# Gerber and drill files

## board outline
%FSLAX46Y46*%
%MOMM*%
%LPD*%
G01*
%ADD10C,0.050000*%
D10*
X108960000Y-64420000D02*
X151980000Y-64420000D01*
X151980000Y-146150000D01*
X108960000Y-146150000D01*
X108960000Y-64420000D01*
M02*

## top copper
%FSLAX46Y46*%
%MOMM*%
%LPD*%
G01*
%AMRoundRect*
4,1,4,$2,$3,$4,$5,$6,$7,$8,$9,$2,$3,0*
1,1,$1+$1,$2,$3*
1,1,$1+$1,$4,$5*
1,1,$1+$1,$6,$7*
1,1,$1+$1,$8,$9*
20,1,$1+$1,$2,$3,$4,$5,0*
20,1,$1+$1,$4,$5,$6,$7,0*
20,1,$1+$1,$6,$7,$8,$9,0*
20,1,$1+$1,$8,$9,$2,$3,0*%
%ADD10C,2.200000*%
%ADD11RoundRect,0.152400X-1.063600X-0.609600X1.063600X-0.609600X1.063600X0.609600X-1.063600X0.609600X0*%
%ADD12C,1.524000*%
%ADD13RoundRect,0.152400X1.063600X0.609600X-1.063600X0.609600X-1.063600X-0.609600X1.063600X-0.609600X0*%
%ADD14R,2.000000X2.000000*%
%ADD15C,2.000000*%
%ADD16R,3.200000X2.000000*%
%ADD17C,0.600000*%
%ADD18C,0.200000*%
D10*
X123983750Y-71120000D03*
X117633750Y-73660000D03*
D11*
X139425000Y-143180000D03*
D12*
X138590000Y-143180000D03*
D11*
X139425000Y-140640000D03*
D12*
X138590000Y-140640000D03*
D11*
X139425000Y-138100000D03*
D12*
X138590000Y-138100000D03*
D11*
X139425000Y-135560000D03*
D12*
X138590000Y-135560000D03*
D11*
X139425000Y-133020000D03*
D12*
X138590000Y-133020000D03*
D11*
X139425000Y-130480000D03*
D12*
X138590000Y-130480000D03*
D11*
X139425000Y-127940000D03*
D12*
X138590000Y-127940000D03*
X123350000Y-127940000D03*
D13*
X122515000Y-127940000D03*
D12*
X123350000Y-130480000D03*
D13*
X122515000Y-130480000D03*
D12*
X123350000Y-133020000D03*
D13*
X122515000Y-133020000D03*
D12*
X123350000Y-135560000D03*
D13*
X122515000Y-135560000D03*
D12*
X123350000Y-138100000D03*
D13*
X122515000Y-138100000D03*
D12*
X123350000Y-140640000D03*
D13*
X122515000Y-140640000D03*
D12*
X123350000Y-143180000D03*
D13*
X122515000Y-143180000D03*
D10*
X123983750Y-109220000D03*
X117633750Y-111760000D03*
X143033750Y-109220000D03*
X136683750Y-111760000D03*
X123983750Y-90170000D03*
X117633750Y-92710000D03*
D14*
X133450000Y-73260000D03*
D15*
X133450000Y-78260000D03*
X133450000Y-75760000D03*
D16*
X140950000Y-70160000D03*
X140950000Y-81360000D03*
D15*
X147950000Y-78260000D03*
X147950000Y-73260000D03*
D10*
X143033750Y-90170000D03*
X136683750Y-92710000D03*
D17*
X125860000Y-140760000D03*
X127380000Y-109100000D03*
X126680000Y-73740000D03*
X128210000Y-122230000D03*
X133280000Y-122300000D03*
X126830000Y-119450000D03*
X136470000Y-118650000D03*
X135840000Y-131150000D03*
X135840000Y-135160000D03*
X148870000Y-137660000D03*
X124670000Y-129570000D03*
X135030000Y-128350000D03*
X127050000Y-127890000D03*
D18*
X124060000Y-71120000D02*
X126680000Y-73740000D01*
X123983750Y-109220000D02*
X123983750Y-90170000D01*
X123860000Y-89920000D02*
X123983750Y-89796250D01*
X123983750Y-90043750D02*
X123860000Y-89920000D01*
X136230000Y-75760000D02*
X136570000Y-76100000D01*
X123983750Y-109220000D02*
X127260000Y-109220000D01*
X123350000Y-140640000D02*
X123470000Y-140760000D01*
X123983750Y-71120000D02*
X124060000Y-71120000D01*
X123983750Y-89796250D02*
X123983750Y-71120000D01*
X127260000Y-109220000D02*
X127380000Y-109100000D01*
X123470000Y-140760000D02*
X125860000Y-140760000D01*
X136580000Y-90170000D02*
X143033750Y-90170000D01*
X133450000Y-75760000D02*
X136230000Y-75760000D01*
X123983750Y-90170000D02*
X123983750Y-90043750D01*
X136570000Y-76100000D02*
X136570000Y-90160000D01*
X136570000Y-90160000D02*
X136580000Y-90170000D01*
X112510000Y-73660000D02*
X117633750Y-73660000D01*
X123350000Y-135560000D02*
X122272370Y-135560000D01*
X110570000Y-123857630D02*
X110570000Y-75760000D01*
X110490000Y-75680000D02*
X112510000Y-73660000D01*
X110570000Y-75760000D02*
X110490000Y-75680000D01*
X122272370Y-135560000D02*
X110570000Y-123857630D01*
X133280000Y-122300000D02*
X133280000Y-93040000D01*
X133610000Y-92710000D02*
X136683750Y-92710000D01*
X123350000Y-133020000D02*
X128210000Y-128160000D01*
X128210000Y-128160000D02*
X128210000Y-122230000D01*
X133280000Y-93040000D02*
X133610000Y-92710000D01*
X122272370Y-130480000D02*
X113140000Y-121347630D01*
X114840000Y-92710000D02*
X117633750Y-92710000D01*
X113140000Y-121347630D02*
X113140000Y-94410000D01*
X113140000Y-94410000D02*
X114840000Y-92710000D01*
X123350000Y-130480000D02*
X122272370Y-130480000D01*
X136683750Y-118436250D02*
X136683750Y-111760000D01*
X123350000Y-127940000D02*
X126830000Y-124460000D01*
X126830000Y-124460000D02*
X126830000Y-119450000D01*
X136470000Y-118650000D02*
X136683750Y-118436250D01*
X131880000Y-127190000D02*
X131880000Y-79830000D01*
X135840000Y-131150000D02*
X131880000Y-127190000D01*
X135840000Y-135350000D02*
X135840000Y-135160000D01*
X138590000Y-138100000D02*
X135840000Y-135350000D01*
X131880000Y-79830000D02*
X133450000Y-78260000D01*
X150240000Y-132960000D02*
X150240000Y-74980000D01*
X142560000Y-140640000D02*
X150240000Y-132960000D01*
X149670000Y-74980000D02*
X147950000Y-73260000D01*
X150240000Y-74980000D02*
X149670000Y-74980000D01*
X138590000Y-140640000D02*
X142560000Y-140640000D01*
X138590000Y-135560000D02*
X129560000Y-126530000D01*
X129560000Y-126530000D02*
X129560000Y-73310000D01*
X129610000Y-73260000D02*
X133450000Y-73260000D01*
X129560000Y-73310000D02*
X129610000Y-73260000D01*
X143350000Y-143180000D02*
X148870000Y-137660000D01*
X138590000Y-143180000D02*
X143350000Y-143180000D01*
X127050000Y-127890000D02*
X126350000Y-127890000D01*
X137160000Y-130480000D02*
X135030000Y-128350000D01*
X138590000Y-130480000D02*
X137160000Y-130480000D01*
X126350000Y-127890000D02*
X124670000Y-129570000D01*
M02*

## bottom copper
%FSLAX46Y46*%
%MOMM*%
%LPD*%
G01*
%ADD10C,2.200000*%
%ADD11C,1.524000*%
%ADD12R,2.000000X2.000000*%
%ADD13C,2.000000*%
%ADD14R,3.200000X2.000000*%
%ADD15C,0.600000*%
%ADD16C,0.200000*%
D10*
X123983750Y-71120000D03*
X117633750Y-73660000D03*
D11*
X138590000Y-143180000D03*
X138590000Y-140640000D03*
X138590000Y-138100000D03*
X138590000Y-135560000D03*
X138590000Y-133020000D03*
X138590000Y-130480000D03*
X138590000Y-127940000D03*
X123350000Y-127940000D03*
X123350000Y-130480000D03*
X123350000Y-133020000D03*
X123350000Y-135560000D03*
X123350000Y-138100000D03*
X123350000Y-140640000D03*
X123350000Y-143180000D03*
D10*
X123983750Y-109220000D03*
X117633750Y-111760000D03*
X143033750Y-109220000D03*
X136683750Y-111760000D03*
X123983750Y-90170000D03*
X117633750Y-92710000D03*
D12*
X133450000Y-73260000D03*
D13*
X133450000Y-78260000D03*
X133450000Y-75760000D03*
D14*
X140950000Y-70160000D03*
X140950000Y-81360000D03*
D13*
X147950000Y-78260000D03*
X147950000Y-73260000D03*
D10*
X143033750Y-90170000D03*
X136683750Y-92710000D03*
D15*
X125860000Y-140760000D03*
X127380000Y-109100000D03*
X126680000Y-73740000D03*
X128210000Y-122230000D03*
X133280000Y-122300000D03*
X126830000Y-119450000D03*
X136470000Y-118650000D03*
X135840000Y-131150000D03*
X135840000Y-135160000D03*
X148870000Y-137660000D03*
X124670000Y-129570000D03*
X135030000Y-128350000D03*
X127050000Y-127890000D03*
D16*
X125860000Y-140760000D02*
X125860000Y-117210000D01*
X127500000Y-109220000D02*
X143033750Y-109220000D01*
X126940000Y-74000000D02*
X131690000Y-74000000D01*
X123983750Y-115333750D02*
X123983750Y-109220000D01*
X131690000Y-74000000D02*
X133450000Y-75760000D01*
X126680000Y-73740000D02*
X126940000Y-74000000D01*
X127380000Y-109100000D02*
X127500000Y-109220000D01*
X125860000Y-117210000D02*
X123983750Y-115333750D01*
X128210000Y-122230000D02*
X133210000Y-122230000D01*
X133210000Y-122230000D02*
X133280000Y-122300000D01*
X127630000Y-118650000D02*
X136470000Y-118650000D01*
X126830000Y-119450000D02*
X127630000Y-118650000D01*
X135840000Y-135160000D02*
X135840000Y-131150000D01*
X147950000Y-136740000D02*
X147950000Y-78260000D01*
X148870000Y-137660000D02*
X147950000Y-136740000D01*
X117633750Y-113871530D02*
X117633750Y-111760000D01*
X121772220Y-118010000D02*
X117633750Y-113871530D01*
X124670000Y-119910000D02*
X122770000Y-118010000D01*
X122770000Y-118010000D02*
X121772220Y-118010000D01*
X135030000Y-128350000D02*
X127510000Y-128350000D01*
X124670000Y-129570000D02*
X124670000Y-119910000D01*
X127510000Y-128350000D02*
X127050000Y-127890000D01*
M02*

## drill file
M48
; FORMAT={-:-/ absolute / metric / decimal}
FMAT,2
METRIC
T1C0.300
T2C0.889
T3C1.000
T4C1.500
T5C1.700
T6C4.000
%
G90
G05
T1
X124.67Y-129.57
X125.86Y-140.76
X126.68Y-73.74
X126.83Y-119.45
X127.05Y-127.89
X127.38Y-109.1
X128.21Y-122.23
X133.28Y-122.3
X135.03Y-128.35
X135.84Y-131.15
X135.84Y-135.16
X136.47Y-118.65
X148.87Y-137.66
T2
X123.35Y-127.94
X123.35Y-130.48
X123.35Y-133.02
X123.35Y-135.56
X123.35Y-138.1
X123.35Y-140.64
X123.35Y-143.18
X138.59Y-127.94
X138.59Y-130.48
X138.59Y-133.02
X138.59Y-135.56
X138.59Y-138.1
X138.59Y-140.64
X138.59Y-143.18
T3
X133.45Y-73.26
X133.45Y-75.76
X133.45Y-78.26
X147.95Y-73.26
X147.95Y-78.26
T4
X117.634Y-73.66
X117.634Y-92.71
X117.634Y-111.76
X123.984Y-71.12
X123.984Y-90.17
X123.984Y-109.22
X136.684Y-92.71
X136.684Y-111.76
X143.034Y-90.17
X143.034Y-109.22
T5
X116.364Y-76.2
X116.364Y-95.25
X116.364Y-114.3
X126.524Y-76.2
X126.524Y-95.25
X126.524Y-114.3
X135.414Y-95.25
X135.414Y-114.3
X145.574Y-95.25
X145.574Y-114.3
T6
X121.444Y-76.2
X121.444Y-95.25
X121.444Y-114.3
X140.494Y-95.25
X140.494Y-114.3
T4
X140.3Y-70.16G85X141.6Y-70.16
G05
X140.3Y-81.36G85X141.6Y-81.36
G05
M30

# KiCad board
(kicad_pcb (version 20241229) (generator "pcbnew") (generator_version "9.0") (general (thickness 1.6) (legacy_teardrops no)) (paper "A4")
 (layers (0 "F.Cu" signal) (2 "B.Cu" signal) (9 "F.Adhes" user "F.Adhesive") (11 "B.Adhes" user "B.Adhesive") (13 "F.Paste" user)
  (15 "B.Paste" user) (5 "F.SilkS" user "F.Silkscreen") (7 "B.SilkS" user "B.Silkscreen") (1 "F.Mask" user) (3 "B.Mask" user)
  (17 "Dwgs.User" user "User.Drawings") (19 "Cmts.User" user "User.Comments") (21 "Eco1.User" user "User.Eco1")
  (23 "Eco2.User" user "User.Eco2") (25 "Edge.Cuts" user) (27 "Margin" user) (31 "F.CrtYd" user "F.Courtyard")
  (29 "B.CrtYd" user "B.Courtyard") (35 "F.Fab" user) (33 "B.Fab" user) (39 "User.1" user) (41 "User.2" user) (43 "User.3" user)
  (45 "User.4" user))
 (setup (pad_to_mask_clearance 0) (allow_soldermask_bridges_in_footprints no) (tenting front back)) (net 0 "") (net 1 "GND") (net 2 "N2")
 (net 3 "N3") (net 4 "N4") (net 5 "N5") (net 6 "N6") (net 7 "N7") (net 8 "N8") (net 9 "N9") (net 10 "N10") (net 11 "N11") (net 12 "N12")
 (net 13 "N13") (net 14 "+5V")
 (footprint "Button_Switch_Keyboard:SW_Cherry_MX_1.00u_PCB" (layer "F.Cu") (at 123.98375 71.12)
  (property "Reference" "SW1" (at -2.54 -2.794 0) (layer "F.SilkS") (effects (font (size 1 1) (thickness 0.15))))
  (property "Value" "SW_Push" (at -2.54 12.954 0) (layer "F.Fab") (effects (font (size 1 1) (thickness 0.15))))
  (pad "" np_thru_hole circle (at -7.62 5.08) (size 1.7 1.7) (drill 1.7) (layers "*.Cu" "*.Mask"))
  (pad "" np_thru_hole circle (at -2.54 5.08) (size 4 4) (drill 4) (layers "*.Cu" "*.Mask"))
  (pad "" np_thru_hole circle (at 2.54 5.08) (size 1.7 1.7) (drill 1.7) (layers "*.Cu" "*.Mask"))
  (pad "1" thru_hole circle (at 0 0) (size 2.2 2.2) (drill 1.5) (layers "*.Cu" "*.Mask") (remove_unused_layers no) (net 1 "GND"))
  (pad "2" thru_hole circle (at -6.35 2.54) (size 2.2 2.2) (drill 1.5) (layers "*.Cu" "*.Mask") (remove_unused_layers no) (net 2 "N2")))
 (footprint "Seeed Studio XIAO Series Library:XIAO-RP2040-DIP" (layer "F.Cu") (at 130.97 135.56 180)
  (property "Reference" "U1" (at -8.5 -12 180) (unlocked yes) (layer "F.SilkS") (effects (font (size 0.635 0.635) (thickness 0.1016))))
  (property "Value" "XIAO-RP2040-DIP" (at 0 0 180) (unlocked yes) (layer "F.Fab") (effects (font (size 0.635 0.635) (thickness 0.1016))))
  (pad "1" smd roundrect (at -8.455 -7.62) (size 2.432 1.524) (layers "F.Cu" "F.Mask") (roundrect_rratio 0.1) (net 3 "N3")
   (thermal_bridge_angle 45))
  (pad "1" thru_hole circle (at -7.62 -7.62) (size 1.524 1.524) (drill 0.889) (layers "*.Cu" "*.Mask") (remove_unused_layers no)
   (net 3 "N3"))
  (pad "2" smd roundrect (at -8.455 -5.08) (size 2.432 1.524) (layers "F.Cu" "F.Mask") (roundrect_rratio 0.1) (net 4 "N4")
   (thermal_bridge_angle 45))
  (pad "2" thru_hole circle (at -7.62 -5.08) (size 1.524 1.524) (drill 0.889) (layers "*.Cu" "*.Mask") (remove_unused_layers no)
   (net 4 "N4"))
  (pad "3" smd roundrect (at -8.455 -2.54) (size 2.432 1.524) (layers "F.Cu" "F.Mask") (roundrect_rratio 0.1) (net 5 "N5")
   (thermal_bridge_angle 45))
  (pad "3" thru_hole circle (at -7.62 -2.54) (size 1.524 1.524) (drill 0.889) (layers "*.Cu" "*.Mask") (remove_unused_layers no)
   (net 5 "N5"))
  (pad "4" smd roundrect (at -8.455 0) (size 2.432 1.524) (layers "F.Cu" "F.Mask") (roundrect_rratio 0.1) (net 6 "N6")
   (thermal_bridge_angle 45))
  (pad "4" thru_hole circle (at -7.62 0) (size 1.524 1.524) (drill 0.889) (layers "*.Cu" "*.Mask") (remove_unused_layers no) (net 6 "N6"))
  (pad "5" smd roundrect (at -8.455 2.54) (size 2.432 1.524) (layers "F.Cu" "F.Mask") (roundrect_rratio 0.1) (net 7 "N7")
   (thermal_bridge_angle 45))
  (pad "5" thru_hole circle (at -7.62 2.54) (size 1.524 1.524) (drill 0.889) (layers "*.Cu" "*.Mask") (remove_unused_layers no) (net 7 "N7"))
  (pad "6" smd roundrect (at -8.455 5.08) (size 2.432 1.524) (layers "F.Cu" "F.Mask") (roundrect_rratio 0.1) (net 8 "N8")
   (thermal_bridge_angle 45))
  (pad "6" thru_hole circle (at -7.62 5.08) (size 1.524 1.524) (drill 0.889) (layers "*.Cu" "*.Mask") (remove_unused_layers no) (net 8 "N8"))
  (pad "7" smd roundrect (at -8.455 7.62) (size 2.432 1.524) (layers "F.Cu" "F.Mask") (roundrect_rratio 0.1) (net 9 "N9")
   (thermal_bridge_angle 45))
  (pad "7" thru_hole circle (at -7.62 7.62) (size 1.524 1.524) (drill 0.889) (layers "*.Cu" "*.Mask") (remove_unused_layers no) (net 9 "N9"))
  (pad "8" thru_hole circle (at 7.62 7.62 180) (size 1.524 1.524) (drill 0.889) (layers "*.Cu" "*.Mask") (remove_unused_layers no)
   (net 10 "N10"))
  (pad "8" smd roundrect (at 8.455 7.62 180) (size 2.432 1.524) (layers "F.Cu" "F.Mask") (roundrect_rratio 0.1) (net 10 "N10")
   (thermal_bridge_angle 45))
  (pad "9" thru_hole circle (at 7.62 5.08 180) (size 1.524 1.524) (drill 0.889) (layers "*.Cu" "*.Mask") (remove_unused_layers no)
   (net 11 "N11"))
  (pad "9" smd roundrect (at 8.455 5.08 180) (size 2.432 1.524) (layers "F.Cu" "F.Mask") (roundrect_rratio 0.1) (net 11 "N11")
   (thermal_bridge_angle 45))
  (pad "10" thru_hole circle (at 7.62 2.54 180) (size 1.524 1.524) (drill 0.889) (layers "*.Cu" "*.Mask") (remove_unused_layers no)
   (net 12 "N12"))
  (pad "10" smd roundrect (at 8.455 2.54 180) (size 2.432 1.524) (layers "F.Cu" "F.Mask") (roundrect_rratio 0.1) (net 12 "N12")
   (thermal_bridge_angle 45))
  (pad "11" thru_hole circle (at 7.62 0 180) (size 1.524 1.524) (drill 0.889) (layers "*.Cu" "*.Mask") (remove_unused_layers no)
   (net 2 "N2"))
  (pad "11" smd roundrect (at 8.455 0 180) (size 2.432 1.524) (layers "F.Cu" "F.Mask") (roundrect_rratio 0.1) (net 2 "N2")
   (thermal_bridge_angle 45))
  (pad "12" thru_hole circle (at 7.62 -2.54 180) (size 1.524 1.524) (drill 0.889) (layers "*.Cu" "*.Mask") (remove_unused_layers no)
   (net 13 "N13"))
  (pad "12" smd roundrect (at 8.455 -2.54 180) (size 2.432 1.524) (layers "F.Cu" "F.Mask") (roundrect_rratio 0.1) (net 13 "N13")
   (thermal_bridge_angle 45))
  (pad "13" thru_hole circle (at 7.62 -5.08 180) (size 1.524 1.524) (drill 0.889) (layers "*.Cu" "*.Mask") (remove_unused_layers no)
   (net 1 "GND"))
  (pad "13" smd roundrect (at 8.455 -5.08 180) (size 2.432 1.524) (layers "F.Cu" "F.Mask") (roundrect_rratio 0.1) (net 1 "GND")
   (thermal_bridge_angle 45))
  (pad "14" thru_hole circle (at 7.62 -7.62 180) (size 1.524 1.524) (drill 0.889) (layers "*.Cu" "*.Mask") (remove_unused_layers no)
   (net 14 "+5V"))
  (pad "14" smd roundrect (at 8.455 -7.62 180) (size 2.432 1.524) (layers "F.Cu" "F.Mask") (roundrect_rratio 0.1) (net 14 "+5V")
   (thermal_bridge_angle 45)))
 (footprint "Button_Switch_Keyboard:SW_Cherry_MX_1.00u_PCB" (layer "F.Cu") (at 123.98375 109.22)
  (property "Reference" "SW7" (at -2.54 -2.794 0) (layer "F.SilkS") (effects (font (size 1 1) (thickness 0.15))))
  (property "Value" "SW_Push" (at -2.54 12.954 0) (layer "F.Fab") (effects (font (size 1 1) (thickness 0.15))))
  (pad "" np_thru_hole circle (at -7.62 5.08) (size 1.7 1.7) (drill 1.7) (layers "*.Cu" "*.Mask"))
  (pad "" np_thru_hole circle (at -2.54 5.08) (size 4 4) (drill 4) (layers "*.Cu" "*.Mask"))
  (pad "" np_thru_hole circle (at 2.54 5.08) (size 1.7 1.7) (drill 1.7) (layers "*.Cu" "*.Mask"))
  (pad "1" thru_hole circle (at 0 0) (size 2.2 2.2) (drill 1.5) (layers "*.Cu" "*.Mask") (remove_unused_layers no) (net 1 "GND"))
  (pad "2" thru_hole circle (at -6.35 2.54) (size 2.2 2.2) (drill 1.5) (layers "*.Cu" "*.Mask") (remove_unused_layers no) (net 8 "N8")))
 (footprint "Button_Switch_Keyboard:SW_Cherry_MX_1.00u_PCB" (layer "F.Cu") (at 143.03375 109.22)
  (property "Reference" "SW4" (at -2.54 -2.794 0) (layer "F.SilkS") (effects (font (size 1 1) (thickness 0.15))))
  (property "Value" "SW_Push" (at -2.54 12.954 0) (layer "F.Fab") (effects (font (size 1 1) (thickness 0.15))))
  (pad "" np_thru_hole circle (at -7.62 5.08) (size 1.7 1.7) (drill 1.7) (layers "*.Cu" "*.Mask"))
  (pad "" np_thru_hole circle (at -2.54 5.08) (size 4 4) (drill 4) (layers "*.Cu" "*.Mask"))
  (pad "" np_thru_hole circle (at 2.54 5.08) (size 1.7 1.7) (drill 1.7) (layers "*.Cu" "*.Mask"))
  (pad "1" thru_hole circle (at 0 0) (size 2.2 2.2) (drill 1.5) (layers "*.Cu" "*.Mask") (remove_unused_layers no) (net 1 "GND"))
  (pad "2" thru_hole circle (at -6.35 2.54) (size 2.2 2.2) (drill 1.5) (layers "*.Cu" "*.Mask") (remove_unused_layers no) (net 10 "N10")))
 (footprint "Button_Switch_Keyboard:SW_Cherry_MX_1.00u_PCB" (layer "F.Cu") (at 123.98375 90.17)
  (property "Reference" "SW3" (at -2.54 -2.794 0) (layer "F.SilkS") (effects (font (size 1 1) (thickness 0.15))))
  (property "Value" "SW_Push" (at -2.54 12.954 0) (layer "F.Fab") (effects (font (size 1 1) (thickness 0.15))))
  (pad "" np_thru_hole circle (at -7.62 5.08) (size 1.7 1.7) (drill 1.7) (layers "*.Cu" "*.Mask"))
  (pad "" np_thru_hole circle (at -2.54 5.08) (size 4 4) (drill 4) (layers "*.Cu" "*.Mask"))
  (pad "" np_thru_hole circle (at 2.54 5.08) (size 1.7 1.7) (drill 1.7) (layers "*.Cu" "*.Mask"))
  (pad "1" thru_hole circle (at 0 0) (size 2.2 2.2) (drill 1.5) (layers "*.Cu" "*.Mask") (remove_unused_layers no) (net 1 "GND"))
  (pad "2" thru_hole circle (at -6.35 2.54) (size 2.2 2.2) (drill 1.5) (layers "*.Cu" "*.Mask") (remove_unused_layers no) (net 11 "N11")))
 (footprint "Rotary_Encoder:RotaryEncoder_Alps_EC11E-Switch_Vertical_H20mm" (layer "F.Cu") (at 133.45 73.26)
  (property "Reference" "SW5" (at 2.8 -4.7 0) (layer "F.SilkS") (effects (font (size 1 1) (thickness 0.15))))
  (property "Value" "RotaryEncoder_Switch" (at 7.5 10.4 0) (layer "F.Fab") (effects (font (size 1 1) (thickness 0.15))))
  (pad "A" thru_hole rect (at 0 0) (size 2 2) (drill 1) (layers "*.Cu" "*.Mask") (remove_unused_layers no) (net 6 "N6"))
  (pad "B" thru_hole circle (at 0 5) (size 2 2) (drill 1) (layers "*.Cu" "*.Mask") (remove_unused_layers no) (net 5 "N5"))
  (pad "C" thru_hole circle (at 0 2.5) (size 2 2) (drill 1) (layers "*.Cu" "*.Mask") (remove_unused_layers no) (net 1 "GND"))
  (pad "MP" thru_hole rect (at 7.5 -3.1) (size 3.2 2) (drill oval 2.8 1.5) (layers "*.Cu" "*.Mask") (remove_unused_layers no))
  (pad "MP" thru_hole rect (at 7.5 8.1) (size 3.2 2) (drill oval 2.8 1.5) (layers "*.Cu" "*.Mask") (remove_unused_layers no))
  (pad "S1" thru_hole circle (at 14.5 5) (size 2 2) (drill 1) (layers "*.Cu" "*.Mask") (remove_unused_layers no) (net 3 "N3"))
  (pad "S2" thru_hole circle (at 14.5 0) (size 2 2) (drill 1) (layers "*.Cu" "*.Mask") (remove_unused_layers no) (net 4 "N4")))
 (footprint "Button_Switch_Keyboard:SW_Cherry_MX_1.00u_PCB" (layer "F.Cu") (at 143.03375 90.17)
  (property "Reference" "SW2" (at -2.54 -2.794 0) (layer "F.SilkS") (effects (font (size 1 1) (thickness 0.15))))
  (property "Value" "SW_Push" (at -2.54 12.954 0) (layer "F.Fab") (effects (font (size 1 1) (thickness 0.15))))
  (pad "" np_thru_hole circle (at -7.62 5.08) (size 1.7 1.7) (drill 1.7) (layers "*.Cu" "*.Mask"))
  (pad "" np_thru_hole circle (at -2.54 5.08) (size 4 4) (drill 4) (layers "*.Cu" "*.Mask"))
  (pad "" np_thru_hole circle (at 2.54 5.08) (size 1.7 1.7) (drill 1.7) (layers "*.Cu" "*.Mask"))
  (pad "1" thru_hole circle (at 0 0) (size 2.2 2.2) (drill 1.5) (layers "*.Cu" "*.Mask") (remove_unused_layers no) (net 1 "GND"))
  (pad "2" thru_hole circle (at -6.35 2.54) (size 2.2 2.2) (drill 1.5) (layers "*.Cu" "*.Mask") (remove_unused_layers no) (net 12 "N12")))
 (gr_rect (start 108.96 64.42) (end 151.98 146.15) (stroke (width 0.05) (type default)) (fill no) (layer "Edge.Cuts"))
 (segment (start 124.06 71.12) (end 126.68 73.74) (width 0.2) (layer "F.Cu") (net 1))
 (segment (start 123.98375 109.22) (end 123.98375 90.17) (width 0.2) (layer "F.Cu") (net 1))
 (segment (start 123.86 89.92) (end 123.98375 89.79625) (width 0.2) (layer "F.Cu") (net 1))
 (segment (start 123.98375 90.04375) (end 123.86 89.92) (width 0.2) (layer "F.Cu") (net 1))
 (segment (start 136.23 75.76) (end 136.57 76.1) (width 0.2) (layer "F.Cu") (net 1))
 (segment (start 123.98375 109.22) (end 127.26 109.22) (width 0.2) (layer "F.Cu") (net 1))
 (segment (start 123.35 140.64) (end 123.47 140.76) (width 0.2) (layer "F.Cu") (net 1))
 (segment (start 123.98375 71.12) (end 124.06 71.12) (width 0.2) (layer "F.Cu") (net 1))
 (segment (start 123.98375 89.79625) (end 123.98375 71.12) (width 0.2) (layer "F.Cu") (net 1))
 (segment (start 127.26 109.22) (end 127.38 109.1) (width 0.2) (layer "F.Cu") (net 1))
 (segment (start 123.47 140.76) (end 125.86 140.76) (width 0.2) (layer "F.Cu") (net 1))
 (segment (start 136.58 90.17) (end 143.03375 90.17) (width 0.2) (layer "F.Cu") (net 1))
 (segment (start 133.45 75.76) (end 136.23 75.76) (width 0.2) (layer "F.Cu") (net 1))
 (segment (start 123.98375 90.17) (end 123.98375 90.04375) (width 0.2) (layer "F.Cu") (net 1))
 (segment (start 136.57 76.1) (end 136.57 90.16) (width 0.2) (layer "F.Cu") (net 1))
 (segment (start 136.57 90.16) (end 136.58 90.17) (width 0.2) (layer "F.Cu") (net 1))
 (via (at 125.86 140.76) (size 0.6) (drill 0.3) (layers "F.Cu" "B.Cu") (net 1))
 (via (at 127.38 109.1) (size 0.6) (drill 0.3) (layers "F.Cu" "B.Cu") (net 1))
 (via (at 126.68 73.74) (size 0.6) (drill 0.3) (layers "F.Cu" "B.Cu") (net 1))
 (segment (start 125.86 140.76) (end 125.86 117.21) (width 0.2) (layer "B.Cu") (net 1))
 (segment (start 127.5 109.22) (end 143.03375 109.22) (width 0.2) (layer "B.Cu") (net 1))
 (segment (start 126.94 74) (end 131.69 74) (width 0.2) (layer "B.Cu") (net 1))
 (segment (start 123.98375 115.33375) (end 123.98375 109.22) (width 0.2) (layer "B.Cu") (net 1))
 (segment (start 131.69 74) (end 133.45 75.76) (width 0.2) (layer "B.Cu") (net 1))
 (segment (start 126.68 73.74) (end 126.94 74) (width 0.2) (layer "B.Cu") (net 1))
 (segment (start 127.38 109.1) (end 127.5 109.22) (width 0.2) (layer "B.Cu") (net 1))
 (segment (start 125.86 117.21) (end 123.98375 115.33375) (width 0.2) (layer "B.Cu") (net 1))
 (segment (start 112.51 73.66) (end 117.63375 73.66) (width 0.2) (layer "F.Cu") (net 2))
 (segment (start 123.35 135.56) (end 122.27237 135.56) (width 0.2) (layer "F.Cu") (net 2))
 (segment (start 110.57 123.85763) (end 110.57 75.76) (width 0.2) (layer "F.Cu") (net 2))
 (segment (start 110.49 75.68) (end 112.51 73.66) (width 0.2) (layer "F.Cu") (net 2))
 (segment (start 110.57 75.76) (end 110.49 75.68) (width 0.2) (layer "F.Cu") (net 2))
 (segment (start 122.27237 135.56) (end 110.57 123.85763) (width 0.2) (layer "F.Cu") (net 2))
 (segment (start 133.28 122.3) (end 133.28 93.04) (width 0.2) (layer "F.Cu") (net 12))
 (segment (start 133.61 92.71) (end 136.68375 92.71) (width 0.2) (layer "F.Cu") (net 12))
 (segment (start 123.35 133.02) (end 128.21 128.16) (width 0.2) (layer "F.Cu") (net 12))
 (segment (start 128.21 128.16) (end 128.21 122.23) (width 0.2) (layer "F.Cu") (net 12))
 (segment (start 133.28 93.04) (end 133.61 92.71) (width 0.2) (layer "F.Cu") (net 12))
 (via (at 128.21 122.23) (size 0.6) (drill 0.3) (layers "F.Cu" "B.Cu") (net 12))
 (via (at 133.28 122.3) (size 0.6) (drill 0.3) (layers "F.Cu" "B.Cu") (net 12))
 (segment (start 128.21 122.23) (end 133.21 122.23) (width 0.2) (layer "B.Cu") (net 12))
 (segment (start 133.21 122.23) (end 133.28 122.3) (width 0.2) (layer "B.Cu") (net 12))
 (segment (start 122.27237 130.48) (end 113.14 121.34763) (width 0.2) (layer "F.Cu") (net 11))
 (segment (start 114.84 92.71) (end 117.63375 92.71) (width 0.2) (layer "F.Cu") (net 11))
 (segment (start 113.14 121.34763) (end 113.14 94.41) (width 0.2) (layer "F.Cu") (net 11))
 (segment (start 113.14 94.41) (end 114.84 92.71) (width 0.2) (layer "F.Cu") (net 11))
 (segment (start 123.35 130.48) (end 122.27237 130.48) (width 0.2) (layer "F.Cu") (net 11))
 (segment (start 136.68375 118.43625) (end 136.68375 111.76) (width 0.2) (layer "F.Cu") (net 10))
 (segment (start 123.35 127.94) (end 126.83 124.46) (width 0.2) (layer "F.Cu") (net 10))
 (segment (start 126.83 124.46) (end 126.83 119.45) (width 0.2) (layer "F.Cu") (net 10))
 (segment (start 136.47 118.65) (end 136.68375 118.43625) (width 0.2) (layer "F.Cu") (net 10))
 (via (at 126.83 119.45) (size 0.6) (drill 0.3) (layers "F.Cu" "B.Cu") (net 10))
 (via (at 136.47 118.65) (size 0.6) (drill 0.3) (layers "F.Cu" "B.Cu") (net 10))
 (segment (start 127.63 118.65) (end 136.47 118.65) (width 0.2) (layer "B.Cu") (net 10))
 (segment (start 126.83 119.45) (end 127.63 118.65) (width 0.2) (layer "B.Cu") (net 10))
 (segment (start 131.88 127.19) (end 131.88 79.83) (width 0.2) (layer "F.Cu") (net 5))
 (segment (start 135.84 131.15) (end 131.88 127.19) (width 0.2) (layer "F.Cu") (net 5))
 (segment (start 135.84 135.35) (end 135.84 135.16) (width 0.2) (layer "F.Cu") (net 5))
 (segment (start 138.59 138.1) (end 135.84 135.35) (width 0.2) (layer "F.Cu") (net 5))
 (segment (start 131.88 79.83) (end 133.45 78.26) (width 0.2) (layer "F.Cu") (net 5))
 (via (at 135.84 131.15) (size 0.6) (drill 0.3) (layers "F.Cu" "B.Cu") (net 5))
 (via (at 135.84 135.16) (size 0.6) (drill 0.3) (layers "F.Cu" "B.Cu") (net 5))
 (segment (start 135.84 135.16) (end 135.84 131.15) (width 0.2) (layer "B.Cu") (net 5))
 (segment (start 150.24 132.96) (end 150.24 74.98) (width 0.2) (layer "F.Cu") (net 4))
 (segment (start 142.56 140.64) (end 150.24 132.96) (width 0.2) (layer "F.Cu") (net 4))
 (segment (start 149.67 74.98) (end 147.95 73.26) (width 0.2) (layer "F.Cu") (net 4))
 (segment (start 150.24 74.98) (end 149.67 74.98) (width 0.2) (layer "F.Cu") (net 4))
 (segment (start 138.59 140.64) (end 142.56 140.64) (width 0.2) (layer "F.Cu") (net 4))
 (segment (start 138.59 135.56) (end 129.56 126.53) (width 0.2) (layer "F.Cu") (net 6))
 (segment (start 129.56 126.53) (end 129.56 73.31) (width 0.2) (layer "F.Cu") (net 6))
 (segment (start 129.61 73.26) (end 133.45 73.26) (width 0.2) (layer "F.Cu") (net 6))
 (segment (start 129.56 73.31) (end 129.61 73.26) (width 0.2) (layer "F.Cu") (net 6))
 (segment (start 143.35 143.18) (end 148.87 137.66) (width 0.2) (layer "F.Cu") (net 3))
 (segment (start 138.59 143.18) (end 143.35 143.18) (width 0.2) (layer "F.Cu") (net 3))
 (via (at 148.87 137.66) (size 0.6) (drill 0.3) (layers "F.Cu" "B.Cu") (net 3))
 (segment (start 147.95 136.74) (end 147.95 78.26) (width 0.2) (layer "B.Cu") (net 3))
 (segment (start 148.87 137.66) (end 147.95 136.74) (width 0.2) (layer "B.Cu") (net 3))
 (segment (start 127.05 127.89) (end 126.35 127.89) (width 0.2) (layer "F.Cu") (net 8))
 (segment (start 137.16 130.48) (end 135.03 128.35) (width 0.2) (layer "F.Cu") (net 8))
 (segment (start 138.59 130.48) (end 137.16 130.48) (width 0.2) (layer "F.Cu") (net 8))
 (segment (start 126.35 127.89) (end 124.67 129.57) (width 0.2) (layer "F.Cu") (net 8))
 (via (at 124.67 129.57) (size 0.6) (drill 0.3) (layers "F.Cu" "B.Cu") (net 8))
 (via (at 135.03 128.35) (size 0.6) (drill 0.3) (layers "F.Cu" "B.Cu") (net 8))
 (via (at 127.05 127.89) (size 0.6) (drill 0.3) (layers "F.Cu" "B.Cu") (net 8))
 (segment (start 117.63375 113.87153) (end 117.63375 111.76) (width 0.2) (layer "B.Cu") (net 8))
 (segment (start 121.77222 118.01) (end 117.63375 113.87153) (width 0.2) (layer "B.Cu") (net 8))
 (segment (start 124.67 119.91) (end 122.77 118.01) (width 0.2) (layer "B.Cu") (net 8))
 (segment (start 122.77 118.01) (end 121.77222 118.01) (width 0.2) (layer "B.Cu") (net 8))
 (segment (start 135.03 128.35) (end 127.51 128.35) (width 0.2) (layer "B.Cu") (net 8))
 (segment (start 124.67 129.57) (end 124.67 119.91) (width 0.2) (layer "B.Cu") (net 8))
 (segment (start 127.51 128.35) (end 127.05 127.89) (width 0.2) (layer "B.Cu") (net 8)))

